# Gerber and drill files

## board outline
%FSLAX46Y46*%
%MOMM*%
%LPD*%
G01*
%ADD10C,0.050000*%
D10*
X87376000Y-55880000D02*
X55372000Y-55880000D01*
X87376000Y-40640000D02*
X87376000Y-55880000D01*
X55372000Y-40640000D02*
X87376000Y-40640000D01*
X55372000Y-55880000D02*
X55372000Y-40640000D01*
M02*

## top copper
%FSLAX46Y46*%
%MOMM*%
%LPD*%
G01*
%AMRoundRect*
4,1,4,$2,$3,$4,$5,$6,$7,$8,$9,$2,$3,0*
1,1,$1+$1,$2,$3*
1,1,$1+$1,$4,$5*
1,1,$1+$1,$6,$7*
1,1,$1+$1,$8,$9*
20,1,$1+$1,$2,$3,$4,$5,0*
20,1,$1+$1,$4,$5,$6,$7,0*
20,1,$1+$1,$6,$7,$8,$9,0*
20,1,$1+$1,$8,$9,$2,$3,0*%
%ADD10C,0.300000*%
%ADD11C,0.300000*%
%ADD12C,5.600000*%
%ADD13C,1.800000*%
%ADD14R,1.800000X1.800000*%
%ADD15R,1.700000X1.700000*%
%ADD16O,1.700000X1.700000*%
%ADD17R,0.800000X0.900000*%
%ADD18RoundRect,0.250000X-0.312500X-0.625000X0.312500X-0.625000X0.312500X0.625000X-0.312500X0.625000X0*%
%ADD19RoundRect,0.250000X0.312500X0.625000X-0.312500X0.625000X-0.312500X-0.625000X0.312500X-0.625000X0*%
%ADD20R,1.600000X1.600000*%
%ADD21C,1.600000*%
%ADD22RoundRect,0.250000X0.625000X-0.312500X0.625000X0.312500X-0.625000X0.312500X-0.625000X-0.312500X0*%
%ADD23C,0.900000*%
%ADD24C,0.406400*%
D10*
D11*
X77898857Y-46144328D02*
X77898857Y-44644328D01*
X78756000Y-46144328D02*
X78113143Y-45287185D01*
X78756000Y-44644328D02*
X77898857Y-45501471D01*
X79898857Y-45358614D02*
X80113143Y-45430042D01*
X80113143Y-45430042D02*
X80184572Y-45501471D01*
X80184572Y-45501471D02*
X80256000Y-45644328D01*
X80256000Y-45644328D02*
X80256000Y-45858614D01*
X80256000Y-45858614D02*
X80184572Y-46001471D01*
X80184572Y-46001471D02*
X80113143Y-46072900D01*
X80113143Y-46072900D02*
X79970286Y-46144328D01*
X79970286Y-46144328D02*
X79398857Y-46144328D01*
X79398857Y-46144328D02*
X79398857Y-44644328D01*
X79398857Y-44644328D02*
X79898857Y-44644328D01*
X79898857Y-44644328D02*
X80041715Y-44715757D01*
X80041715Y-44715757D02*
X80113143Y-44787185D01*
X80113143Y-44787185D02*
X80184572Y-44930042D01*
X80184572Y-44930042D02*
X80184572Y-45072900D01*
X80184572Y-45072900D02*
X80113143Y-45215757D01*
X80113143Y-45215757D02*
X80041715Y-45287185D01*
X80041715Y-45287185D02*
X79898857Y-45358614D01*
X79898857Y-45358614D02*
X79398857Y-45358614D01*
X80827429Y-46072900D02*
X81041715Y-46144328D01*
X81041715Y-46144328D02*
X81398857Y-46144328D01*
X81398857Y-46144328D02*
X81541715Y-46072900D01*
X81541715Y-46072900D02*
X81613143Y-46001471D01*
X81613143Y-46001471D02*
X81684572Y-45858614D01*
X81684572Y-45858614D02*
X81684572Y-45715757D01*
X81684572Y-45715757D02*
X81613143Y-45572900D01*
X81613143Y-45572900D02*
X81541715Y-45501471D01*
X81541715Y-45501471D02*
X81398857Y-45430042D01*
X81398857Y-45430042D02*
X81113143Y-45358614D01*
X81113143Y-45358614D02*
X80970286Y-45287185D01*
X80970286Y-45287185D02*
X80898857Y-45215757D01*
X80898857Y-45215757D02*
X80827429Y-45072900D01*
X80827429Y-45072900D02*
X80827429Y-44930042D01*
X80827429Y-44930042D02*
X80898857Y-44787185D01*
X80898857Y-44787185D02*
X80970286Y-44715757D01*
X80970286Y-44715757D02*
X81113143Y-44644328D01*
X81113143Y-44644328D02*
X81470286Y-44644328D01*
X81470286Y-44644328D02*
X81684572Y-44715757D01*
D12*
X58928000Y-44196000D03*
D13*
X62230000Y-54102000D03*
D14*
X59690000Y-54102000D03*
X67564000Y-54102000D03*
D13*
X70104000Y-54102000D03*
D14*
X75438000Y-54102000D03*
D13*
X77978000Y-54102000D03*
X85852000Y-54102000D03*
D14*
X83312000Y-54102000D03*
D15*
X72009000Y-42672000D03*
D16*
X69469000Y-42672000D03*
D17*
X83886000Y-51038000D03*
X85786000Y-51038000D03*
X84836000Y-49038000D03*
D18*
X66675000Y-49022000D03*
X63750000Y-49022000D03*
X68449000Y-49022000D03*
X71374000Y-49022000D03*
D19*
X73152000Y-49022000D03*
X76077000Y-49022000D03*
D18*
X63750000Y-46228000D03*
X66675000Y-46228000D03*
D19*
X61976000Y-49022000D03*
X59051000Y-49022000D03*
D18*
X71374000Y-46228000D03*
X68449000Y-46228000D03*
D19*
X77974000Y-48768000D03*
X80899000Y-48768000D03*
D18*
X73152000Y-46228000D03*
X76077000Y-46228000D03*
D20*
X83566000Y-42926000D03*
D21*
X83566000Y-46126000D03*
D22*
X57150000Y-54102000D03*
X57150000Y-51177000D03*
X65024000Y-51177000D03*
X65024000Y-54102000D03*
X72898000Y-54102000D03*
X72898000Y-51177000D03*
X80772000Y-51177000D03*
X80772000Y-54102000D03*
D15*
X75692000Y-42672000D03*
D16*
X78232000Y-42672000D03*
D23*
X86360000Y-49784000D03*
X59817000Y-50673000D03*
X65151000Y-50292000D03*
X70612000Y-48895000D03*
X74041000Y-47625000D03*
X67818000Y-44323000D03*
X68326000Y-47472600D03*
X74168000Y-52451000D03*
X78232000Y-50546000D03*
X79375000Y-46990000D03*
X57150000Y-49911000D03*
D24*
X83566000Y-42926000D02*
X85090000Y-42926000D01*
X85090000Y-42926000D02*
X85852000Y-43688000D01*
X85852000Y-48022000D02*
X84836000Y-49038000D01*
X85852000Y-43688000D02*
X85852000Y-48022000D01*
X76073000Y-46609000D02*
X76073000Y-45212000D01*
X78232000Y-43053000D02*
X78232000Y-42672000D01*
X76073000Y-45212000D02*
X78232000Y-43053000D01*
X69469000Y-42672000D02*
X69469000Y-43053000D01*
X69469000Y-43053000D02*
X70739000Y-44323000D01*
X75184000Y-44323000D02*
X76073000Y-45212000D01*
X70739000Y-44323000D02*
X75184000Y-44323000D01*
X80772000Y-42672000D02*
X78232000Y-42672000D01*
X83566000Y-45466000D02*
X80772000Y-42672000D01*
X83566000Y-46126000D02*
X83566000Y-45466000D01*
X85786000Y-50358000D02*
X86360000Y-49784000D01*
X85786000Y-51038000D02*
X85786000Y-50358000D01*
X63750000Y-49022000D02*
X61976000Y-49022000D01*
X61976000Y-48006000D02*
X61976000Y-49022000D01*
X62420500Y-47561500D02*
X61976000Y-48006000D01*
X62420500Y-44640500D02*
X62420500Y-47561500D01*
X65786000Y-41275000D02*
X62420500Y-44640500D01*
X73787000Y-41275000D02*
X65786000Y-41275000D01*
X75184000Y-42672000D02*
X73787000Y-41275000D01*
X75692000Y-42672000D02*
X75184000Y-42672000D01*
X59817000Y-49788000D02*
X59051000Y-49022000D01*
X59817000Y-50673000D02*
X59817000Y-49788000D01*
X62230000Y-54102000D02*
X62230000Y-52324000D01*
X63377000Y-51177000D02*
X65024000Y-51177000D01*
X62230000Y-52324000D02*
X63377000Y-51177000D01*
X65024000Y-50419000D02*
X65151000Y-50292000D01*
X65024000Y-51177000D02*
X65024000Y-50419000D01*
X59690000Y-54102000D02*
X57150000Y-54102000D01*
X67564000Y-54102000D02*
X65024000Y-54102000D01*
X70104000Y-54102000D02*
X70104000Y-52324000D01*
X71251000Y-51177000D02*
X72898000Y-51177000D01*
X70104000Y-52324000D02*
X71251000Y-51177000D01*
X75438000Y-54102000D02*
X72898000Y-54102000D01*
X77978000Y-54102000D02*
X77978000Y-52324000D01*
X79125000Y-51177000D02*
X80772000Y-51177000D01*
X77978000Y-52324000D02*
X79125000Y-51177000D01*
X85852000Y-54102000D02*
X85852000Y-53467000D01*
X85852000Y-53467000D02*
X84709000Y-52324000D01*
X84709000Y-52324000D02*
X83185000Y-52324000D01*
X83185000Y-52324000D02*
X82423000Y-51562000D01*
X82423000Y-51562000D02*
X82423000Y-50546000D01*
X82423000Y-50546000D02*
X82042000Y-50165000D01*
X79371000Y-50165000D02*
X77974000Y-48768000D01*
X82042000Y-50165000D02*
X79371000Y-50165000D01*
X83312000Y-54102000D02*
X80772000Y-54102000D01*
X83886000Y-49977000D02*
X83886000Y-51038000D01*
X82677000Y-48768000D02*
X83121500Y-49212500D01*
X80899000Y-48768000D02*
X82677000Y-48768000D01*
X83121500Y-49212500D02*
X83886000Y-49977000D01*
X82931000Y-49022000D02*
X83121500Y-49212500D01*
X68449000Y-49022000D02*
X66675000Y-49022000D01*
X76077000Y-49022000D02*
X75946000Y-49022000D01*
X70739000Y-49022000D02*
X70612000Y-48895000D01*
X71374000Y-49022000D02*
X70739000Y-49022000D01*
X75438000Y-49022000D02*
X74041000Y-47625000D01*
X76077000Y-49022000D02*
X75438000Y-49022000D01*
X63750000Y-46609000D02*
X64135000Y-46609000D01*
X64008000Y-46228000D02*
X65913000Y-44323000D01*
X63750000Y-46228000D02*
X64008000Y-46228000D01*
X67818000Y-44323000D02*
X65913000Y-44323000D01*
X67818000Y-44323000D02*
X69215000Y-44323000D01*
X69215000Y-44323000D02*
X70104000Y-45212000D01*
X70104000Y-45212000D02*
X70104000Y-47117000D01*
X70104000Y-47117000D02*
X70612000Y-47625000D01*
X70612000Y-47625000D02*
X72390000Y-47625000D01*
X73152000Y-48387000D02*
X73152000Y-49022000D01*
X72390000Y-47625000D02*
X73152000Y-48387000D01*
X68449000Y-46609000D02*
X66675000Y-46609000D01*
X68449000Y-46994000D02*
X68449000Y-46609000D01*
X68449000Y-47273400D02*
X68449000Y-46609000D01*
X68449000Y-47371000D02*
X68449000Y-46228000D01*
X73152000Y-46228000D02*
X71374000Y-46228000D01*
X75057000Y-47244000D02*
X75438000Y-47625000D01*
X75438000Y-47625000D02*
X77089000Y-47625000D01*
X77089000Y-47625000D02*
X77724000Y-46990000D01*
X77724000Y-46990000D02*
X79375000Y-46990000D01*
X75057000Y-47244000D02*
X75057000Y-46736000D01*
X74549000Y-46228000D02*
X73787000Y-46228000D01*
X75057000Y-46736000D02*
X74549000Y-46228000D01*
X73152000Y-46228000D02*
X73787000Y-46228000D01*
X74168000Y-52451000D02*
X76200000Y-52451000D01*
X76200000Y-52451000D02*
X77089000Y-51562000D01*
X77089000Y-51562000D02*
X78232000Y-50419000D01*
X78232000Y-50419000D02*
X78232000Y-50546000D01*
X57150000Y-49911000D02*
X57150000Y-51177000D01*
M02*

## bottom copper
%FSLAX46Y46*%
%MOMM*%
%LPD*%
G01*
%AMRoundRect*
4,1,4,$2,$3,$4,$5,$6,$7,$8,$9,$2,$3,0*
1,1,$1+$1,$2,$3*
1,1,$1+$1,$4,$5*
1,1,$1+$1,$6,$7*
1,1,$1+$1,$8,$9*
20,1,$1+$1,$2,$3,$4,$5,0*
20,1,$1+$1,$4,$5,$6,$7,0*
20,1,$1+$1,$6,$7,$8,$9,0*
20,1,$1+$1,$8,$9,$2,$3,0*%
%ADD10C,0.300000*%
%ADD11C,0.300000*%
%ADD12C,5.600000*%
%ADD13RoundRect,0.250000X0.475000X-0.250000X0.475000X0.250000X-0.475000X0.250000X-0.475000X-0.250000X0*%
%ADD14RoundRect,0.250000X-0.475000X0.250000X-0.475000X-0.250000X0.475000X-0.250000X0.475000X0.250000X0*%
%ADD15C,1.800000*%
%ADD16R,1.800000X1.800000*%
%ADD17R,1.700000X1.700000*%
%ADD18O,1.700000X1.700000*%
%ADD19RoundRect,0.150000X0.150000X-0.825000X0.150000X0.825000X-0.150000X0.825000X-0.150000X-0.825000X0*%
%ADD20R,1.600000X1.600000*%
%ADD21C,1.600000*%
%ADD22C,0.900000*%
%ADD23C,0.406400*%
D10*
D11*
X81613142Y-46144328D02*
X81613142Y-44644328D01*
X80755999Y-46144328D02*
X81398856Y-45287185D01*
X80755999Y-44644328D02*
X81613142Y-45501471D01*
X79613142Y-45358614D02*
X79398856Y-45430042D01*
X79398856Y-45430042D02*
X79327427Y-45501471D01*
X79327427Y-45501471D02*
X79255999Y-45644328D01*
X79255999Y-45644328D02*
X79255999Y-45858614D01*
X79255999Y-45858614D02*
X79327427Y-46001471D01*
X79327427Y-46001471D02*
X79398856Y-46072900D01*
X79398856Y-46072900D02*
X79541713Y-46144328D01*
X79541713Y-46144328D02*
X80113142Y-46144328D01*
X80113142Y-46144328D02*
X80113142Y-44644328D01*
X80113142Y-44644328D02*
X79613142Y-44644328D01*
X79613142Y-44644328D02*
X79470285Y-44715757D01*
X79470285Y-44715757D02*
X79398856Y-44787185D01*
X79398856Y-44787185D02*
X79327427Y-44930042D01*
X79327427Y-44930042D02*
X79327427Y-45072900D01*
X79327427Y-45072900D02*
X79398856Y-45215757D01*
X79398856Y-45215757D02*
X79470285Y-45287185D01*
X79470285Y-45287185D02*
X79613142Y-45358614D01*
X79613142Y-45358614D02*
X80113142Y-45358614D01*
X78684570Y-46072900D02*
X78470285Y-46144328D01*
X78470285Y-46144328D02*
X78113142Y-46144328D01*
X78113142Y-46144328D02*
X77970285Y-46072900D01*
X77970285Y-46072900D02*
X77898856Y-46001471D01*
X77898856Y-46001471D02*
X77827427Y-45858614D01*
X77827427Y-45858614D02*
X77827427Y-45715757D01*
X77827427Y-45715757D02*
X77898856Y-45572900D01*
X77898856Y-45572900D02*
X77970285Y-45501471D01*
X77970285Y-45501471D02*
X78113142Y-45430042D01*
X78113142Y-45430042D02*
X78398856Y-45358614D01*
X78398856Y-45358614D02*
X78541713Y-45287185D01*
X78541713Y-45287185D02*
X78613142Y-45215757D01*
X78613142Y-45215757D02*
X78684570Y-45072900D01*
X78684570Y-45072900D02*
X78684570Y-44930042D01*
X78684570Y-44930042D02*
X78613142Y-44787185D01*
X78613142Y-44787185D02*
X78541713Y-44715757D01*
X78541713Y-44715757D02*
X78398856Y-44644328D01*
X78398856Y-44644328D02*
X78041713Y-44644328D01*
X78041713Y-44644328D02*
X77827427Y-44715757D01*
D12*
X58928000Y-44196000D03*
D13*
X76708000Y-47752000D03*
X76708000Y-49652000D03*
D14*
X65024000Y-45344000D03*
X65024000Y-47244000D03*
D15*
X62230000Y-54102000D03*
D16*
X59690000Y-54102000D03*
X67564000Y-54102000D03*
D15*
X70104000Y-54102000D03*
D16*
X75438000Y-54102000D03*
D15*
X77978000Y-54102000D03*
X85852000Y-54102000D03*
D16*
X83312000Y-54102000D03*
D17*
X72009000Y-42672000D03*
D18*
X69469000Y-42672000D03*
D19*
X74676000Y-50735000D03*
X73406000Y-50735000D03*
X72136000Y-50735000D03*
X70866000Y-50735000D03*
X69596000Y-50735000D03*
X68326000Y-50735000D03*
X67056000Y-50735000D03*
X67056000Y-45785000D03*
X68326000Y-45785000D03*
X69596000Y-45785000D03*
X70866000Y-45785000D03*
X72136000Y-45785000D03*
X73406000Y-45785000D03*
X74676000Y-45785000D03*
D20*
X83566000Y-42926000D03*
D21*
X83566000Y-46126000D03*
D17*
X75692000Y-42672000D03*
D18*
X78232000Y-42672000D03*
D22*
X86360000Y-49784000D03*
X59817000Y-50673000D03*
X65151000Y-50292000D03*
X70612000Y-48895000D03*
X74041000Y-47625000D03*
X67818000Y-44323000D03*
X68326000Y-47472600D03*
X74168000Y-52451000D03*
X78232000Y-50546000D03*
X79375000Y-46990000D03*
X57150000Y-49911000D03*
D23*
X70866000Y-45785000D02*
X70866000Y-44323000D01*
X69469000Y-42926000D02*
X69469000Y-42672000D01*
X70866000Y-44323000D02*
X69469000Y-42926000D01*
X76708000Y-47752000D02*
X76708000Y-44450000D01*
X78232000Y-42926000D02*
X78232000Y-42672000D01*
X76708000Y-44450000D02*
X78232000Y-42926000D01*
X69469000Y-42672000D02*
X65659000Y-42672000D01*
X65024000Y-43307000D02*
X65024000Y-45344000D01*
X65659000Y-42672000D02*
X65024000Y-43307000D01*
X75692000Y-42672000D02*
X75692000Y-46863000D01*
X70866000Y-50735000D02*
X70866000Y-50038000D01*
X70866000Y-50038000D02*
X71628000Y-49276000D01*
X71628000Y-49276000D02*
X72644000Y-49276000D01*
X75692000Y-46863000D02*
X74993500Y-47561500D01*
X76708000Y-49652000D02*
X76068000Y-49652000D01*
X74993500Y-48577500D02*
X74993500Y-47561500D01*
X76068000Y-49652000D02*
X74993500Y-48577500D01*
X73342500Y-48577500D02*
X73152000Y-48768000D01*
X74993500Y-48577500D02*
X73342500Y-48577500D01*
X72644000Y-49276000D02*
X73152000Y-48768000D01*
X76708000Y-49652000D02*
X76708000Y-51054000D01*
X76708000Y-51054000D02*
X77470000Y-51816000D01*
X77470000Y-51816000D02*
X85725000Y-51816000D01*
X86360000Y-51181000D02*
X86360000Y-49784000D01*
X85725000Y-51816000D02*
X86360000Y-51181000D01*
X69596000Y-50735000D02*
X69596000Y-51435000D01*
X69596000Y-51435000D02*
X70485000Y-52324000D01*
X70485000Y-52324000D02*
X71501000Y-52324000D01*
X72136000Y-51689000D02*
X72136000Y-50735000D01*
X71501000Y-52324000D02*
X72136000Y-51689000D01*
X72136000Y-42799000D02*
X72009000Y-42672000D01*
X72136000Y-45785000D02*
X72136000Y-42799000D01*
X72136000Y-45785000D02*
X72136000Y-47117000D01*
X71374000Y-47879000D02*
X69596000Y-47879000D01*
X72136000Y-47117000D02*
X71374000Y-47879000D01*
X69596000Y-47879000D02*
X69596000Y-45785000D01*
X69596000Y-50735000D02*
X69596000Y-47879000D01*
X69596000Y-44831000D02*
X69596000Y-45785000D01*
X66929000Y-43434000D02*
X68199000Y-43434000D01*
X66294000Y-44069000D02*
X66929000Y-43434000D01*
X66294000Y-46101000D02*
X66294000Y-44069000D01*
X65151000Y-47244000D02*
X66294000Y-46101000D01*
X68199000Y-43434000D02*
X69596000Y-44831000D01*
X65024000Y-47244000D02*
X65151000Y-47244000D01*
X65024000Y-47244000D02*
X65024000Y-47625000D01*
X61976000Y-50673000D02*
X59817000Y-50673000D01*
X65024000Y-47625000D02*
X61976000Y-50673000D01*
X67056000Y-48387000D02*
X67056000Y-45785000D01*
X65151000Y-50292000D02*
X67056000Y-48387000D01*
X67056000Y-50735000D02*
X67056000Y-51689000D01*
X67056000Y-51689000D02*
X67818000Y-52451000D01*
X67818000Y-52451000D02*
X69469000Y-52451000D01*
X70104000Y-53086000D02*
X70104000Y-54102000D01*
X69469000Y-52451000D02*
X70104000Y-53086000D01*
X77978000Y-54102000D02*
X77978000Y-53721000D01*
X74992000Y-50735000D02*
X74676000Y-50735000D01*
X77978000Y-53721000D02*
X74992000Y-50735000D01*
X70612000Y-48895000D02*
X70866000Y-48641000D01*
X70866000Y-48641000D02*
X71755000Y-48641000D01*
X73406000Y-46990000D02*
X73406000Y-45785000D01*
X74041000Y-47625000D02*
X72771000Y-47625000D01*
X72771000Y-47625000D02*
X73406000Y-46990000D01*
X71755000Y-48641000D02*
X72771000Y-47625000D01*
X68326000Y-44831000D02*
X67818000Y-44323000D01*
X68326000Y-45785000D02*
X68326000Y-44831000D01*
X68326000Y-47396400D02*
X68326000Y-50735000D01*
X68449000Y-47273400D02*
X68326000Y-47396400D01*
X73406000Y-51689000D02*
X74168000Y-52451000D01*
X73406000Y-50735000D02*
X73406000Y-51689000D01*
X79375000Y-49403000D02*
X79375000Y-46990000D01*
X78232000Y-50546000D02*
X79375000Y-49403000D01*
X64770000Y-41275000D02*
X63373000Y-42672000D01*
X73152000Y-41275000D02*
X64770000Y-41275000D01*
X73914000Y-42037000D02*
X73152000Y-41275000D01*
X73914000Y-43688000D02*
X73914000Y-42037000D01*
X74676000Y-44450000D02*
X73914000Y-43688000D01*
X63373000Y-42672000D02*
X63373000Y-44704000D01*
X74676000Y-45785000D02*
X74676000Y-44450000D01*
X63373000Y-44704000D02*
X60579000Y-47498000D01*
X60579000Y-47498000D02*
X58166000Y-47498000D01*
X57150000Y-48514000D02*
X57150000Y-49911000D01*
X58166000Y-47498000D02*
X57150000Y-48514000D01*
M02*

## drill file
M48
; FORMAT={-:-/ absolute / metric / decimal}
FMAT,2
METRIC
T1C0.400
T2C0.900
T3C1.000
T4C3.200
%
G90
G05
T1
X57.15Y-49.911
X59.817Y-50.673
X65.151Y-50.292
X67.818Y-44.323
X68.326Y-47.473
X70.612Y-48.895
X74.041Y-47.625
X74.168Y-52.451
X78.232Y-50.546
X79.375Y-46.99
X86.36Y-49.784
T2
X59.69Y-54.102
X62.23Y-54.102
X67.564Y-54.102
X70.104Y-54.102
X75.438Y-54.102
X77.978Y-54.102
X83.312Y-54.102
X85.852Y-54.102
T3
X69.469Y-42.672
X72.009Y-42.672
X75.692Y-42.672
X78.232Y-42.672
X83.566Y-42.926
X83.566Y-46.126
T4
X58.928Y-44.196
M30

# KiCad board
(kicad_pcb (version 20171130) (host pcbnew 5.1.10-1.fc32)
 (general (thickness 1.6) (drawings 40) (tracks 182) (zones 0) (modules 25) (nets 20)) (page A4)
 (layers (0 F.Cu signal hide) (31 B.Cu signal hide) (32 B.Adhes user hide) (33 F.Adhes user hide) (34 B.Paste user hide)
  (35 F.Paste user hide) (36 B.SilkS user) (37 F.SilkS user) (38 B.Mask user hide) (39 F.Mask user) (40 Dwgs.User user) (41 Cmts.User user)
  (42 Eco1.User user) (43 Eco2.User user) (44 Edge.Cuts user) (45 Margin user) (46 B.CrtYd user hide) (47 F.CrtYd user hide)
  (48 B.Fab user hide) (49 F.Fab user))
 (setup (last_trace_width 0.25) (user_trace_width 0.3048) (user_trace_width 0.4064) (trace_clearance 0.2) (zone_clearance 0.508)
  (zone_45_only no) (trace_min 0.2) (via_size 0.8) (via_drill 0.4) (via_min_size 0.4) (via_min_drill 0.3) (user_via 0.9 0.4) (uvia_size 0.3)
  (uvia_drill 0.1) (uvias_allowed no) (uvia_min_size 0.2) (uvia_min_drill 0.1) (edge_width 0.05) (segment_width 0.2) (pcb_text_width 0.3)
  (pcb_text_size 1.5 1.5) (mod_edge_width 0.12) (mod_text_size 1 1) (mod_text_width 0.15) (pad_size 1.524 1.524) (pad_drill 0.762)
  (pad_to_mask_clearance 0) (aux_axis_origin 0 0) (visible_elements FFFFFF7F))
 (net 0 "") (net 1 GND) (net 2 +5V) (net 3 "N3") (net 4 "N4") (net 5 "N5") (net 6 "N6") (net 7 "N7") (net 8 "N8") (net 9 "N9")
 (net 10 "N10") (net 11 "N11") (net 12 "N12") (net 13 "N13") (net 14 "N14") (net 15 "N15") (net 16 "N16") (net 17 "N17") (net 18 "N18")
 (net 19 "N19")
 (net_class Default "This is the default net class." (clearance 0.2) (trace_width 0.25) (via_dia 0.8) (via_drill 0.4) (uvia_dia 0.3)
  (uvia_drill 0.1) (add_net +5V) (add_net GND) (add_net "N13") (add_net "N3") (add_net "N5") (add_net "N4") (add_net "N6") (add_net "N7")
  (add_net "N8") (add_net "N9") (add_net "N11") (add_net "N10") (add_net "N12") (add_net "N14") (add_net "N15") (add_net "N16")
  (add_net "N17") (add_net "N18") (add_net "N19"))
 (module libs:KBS (layer B.Cu) (at 60.071 48.895 180)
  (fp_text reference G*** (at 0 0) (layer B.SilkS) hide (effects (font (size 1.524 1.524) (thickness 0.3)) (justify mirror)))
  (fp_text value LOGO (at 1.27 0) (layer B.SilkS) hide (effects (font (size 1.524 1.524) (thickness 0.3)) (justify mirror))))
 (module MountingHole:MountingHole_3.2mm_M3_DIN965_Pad (layer F.Cu) (at 58.928 44.196)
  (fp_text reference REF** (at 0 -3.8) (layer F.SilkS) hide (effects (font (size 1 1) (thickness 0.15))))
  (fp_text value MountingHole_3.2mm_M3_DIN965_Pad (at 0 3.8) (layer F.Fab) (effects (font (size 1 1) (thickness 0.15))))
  (pad 1 thru_hole circle (at 0 0) (size 5.6 5.6) (drill 3.2) (layers *.Cu *.Mask)))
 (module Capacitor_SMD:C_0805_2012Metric (layer B.Cu) (at 76.708 48.702 90)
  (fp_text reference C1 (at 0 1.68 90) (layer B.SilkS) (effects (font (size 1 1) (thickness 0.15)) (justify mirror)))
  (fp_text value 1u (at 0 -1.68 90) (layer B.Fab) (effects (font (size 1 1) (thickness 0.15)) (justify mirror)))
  (pad 2 smd roundrect (at 0.95 0 90) (size 1 1.45) (layers B.Cu B.Paste B.Mask) (roundrect_rratio 0.25) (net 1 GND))
  (pad 1 smd roundrect (at -0.95 0 90) (size 1 1.45) (layers B.Cu B.Paste B.Mask) (roundrect_rratio 0.25) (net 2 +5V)))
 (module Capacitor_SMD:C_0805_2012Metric (layer B.Cu) (at 65.024 46.294 270)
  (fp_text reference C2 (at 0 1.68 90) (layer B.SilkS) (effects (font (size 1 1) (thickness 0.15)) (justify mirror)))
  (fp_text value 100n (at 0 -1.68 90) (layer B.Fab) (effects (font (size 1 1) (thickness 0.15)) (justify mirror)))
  (pad 1 smd roundrect (at -0.95 0 270) (size 1 1.45) (layers B.Cu B.Paste B.Mask) (roundrect_rratio 0.25) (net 1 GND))
  (pad 2 smd roundrect (at 0.95 0 270) (size 1 1.45) (layers B.Cu B.Paste B.Mask) (roundrect_rratio 0.25) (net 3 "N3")))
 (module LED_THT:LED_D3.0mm (layer F.Cu) (at 59.69 54.102)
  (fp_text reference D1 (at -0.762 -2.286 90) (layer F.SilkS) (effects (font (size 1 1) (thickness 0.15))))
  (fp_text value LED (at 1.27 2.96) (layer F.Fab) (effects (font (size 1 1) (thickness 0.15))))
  (pad 2 thru_hole circle (at 2.54 0) (size 1.8 1.8) (drill 0.9) (layers *.Cu *.Mask) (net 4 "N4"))
  (pad 1 thru_hole rect (at 0 0) (size 1.8 1.8) (drill 0.9) (layers *.Cu *.Mask) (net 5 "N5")))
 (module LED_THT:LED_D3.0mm (layer F.Cu) (at 67.564 54.102)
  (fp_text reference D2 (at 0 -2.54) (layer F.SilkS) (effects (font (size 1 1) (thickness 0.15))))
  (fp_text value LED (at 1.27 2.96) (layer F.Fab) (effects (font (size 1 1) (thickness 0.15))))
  (pad 1 thru_hole rect (at 0 0) (size 1.8 1.8) (drill 0.9) (layers *.Cu *.Mask) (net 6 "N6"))
  (pad 2 thru_hole circle (at 2.54 0) (size 1.8 1.8) (drill 0.9) (layers *.Cu *.Mask) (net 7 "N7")))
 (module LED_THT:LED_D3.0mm (layer F.Cu) (at 75.438 54.102)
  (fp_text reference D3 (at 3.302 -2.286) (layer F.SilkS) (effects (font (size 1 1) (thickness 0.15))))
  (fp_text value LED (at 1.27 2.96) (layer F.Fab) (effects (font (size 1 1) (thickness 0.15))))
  (pad 1 thru_hole rect (at 0 0) (size 1.8 1.8) (drill 0.9) (layers *.Cu *.Mask) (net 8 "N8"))
  (pad 2 thru_hole circle (at 2.54 0) (size 1.8 1.8) (drill 0.9) (layers *.Cu *.Mask) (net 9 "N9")))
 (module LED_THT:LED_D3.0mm (layer F.Cu) (at 83.312 54.102)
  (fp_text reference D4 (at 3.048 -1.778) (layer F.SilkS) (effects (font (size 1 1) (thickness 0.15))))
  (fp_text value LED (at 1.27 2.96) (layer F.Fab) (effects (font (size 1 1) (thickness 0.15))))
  (pad 2 thru_hole circle (at 2.54 0) (size 1.8 1.8) (drill 0.9) (layers *.Cu *.Mask) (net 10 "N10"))
  (pad 1 thru_hole rect (at 0 0) (size 1.8 1.8) (drill 0.9) (layers *.Cu *.Mask) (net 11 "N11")))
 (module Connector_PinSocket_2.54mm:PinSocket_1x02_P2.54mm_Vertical (layer F.Cu) (at 72.009 42.672 270)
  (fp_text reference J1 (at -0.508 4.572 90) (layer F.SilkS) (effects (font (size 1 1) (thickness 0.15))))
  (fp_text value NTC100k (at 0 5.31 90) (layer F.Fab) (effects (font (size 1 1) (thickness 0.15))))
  (pad 1 thru_hole rect (at 0 0 270) (size 1.7 1.7) (drill 1) (layers *.Cu *.Mask) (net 3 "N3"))
  (pad 2 thru_hole oval (at 0 2.54 270) (size 1.7 1.7) (drill 1) (layers *.Cu *.Mask) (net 1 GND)))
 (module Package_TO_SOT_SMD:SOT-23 (layer F.Cu) (at 84.836 50.038 90)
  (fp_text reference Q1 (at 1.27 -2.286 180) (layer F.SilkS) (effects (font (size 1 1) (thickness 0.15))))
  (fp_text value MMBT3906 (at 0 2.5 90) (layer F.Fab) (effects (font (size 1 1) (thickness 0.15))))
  (pad 1 smd rect (at -1 -0.95 90) (size 0.9 0.8) (layers F.Cu F.Paste F.Mask) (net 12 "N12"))
  (pad 2 smd rect (at -1 0.95 90) (size 0.9 0.8) (layers F.Cu F.Paste F.Mask) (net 2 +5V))
  (pad 3 smd rect (at 1 0 90) (size 0.9 0.8) (layers F.Cu F.Paste F.Mask) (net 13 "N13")))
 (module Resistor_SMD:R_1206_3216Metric (layer F.Cu) (at 65.2125 49.022)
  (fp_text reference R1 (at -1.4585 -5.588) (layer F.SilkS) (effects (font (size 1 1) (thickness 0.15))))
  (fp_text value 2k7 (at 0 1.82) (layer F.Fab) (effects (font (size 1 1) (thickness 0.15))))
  (pad 2 smd roundrect (at 1.4625 0) (size 1.125 1.75) (layers F.Cu F.Paste F.Mask) (roundrect_rratio 0.222222) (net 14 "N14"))
  (pad 1 smd roundrect (at -1.4625 0) (size 1.125 1.75) (layers F.Cu F.Paste F.Mask) (roundrect_rratio 0.222222) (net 2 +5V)))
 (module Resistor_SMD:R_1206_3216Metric (layer F.Cu) (at 69.9115 49.022)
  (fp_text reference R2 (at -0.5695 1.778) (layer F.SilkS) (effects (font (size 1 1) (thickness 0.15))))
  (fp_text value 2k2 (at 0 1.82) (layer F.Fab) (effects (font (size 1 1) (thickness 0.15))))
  (pad 1 smd roundrect (at -1.4625 0) (size 1.125 1.75) (layers F.Cu F.Paste F.Mask) (roundrect_rratio 0.222222) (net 14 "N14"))
  (pad 2 smd roundrect (at 1.4625 0) (size 1.125 1.75) (layers F.Cu F.Paste F.Mask) (roundrect_rratio 0.222222) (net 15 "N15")))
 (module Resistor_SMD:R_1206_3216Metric (layer F.Cu) (at 74.6145 49.022 180)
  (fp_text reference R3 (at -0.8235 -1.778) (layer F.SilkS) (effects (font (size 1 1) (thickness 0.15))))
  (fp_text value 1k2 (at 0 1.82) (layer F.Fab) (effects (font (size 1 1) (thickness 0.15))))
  (pad 2 smd roundrect (at 1.4625 0 180) (size 1.125 1.75) (layers F.Cu F.Paste F.Mask) (roundrect_rratio 0.222222) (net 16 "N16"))
  (pad 1 smd roundrect (at -1.4625 0 180) (size 1.125 1.75) (layers F.Cu F.Paste F.Mask) (roundrect_rratio 0.222222) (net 15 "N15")))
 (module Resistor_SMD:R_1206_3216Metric (layer F.Cu) (at 65.2125 46.228)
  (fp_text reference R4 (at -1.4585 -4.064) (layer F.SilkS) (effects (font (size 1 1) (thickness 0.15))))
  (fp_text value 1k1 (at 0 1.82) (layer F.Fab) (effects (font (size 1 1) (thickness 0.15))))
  (pad 1 smd roundrect (at -1.4625 0) (size 1.125 1.75) (layers F.Cu F.Paste F.Mask) (roundrect_rratio 0.222222) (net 16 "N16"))
  (pad 2 smd roundrect (at 1.4625 0) (size 1.125 1.75) (layers F.Cu F.Paste F.Mask) (roundrect_rratio 0.222222) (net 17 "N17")))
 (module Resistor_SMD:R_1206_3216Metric (layer F.Cu) (at 60.5135 49.022 180)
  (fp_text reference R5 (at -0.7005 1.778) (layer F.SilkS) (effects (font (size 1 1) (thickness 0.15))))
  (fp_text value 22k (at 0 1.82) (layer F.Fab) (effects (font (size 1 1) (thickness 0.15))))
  (pad 1 smd roundrect (at -1.4625 0 180) (size 1.125 1.75) (layers F.Cu F.Paste F.Mask) (roundrect_rratio 0.222222) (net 2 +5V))
  (pad 2 smd roundrect (at 1.4625 0 180) (size 1.125 1.75) (layers F.Cu F.Paste F.Mask) (roundrect_rratio 0.222222) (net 3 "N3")))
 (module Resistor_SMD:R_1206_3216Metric (layer F.Cu) (at 69.9115 46.228)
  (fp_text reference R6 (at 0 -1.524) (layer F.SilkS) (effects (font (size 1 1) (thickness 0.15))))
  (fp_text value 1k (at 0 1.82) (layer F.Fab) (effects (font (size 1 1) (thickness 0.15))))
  (pad 2 smd roundrect (at 1.4625 0) (size 1.125 1.75) (layers F.Cu F.Paste F.Mask) (roundrect_rratio 0.222222) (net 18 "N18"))
  (pad 1 smd roundrect (at -1.4625 0) (size 1.125 1.75) (layers F.Cu F.Paste F.Mask) (roundrect_rratio 0.222222) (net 17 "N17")))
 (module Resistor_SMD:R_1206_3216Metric (layer F.Cu) (at 79.4365 48.768 180)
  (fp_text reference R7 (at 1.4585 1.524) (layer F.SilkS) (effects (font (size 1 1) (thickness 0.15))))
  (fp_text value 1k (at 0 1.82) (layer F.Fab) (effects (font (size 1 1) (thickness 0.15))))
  (pad 2 smd roundrect (at 1.4625 0 180) (size 1.125 1.75) (layers F.Cu F.Paste F.Mask) (roundrect_rratio 0.222222) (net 10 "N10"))
  (pad 1 smd roundrect (at -1.4625 0 180) (size 1.125 1.75) (layers F.Cu F.Paste F.Mask) (roundrect_rratio 0.222222) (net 12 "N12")))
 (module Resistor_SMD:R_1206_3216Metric (layer F.Cu) (at 74.6145 46.228)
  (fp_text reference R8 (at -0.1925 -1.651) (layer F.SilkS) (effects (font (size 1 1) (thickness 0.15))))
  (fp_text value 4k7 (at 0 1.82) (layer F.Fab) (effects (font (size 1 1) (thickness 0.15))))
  (pad 1 smd roundrect (at -1.4625 0) (size 1.125 1.75) (layers F.Cu F.Paste F.Mask) (roundrect_rratio 0.222222) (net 18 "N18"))
  (pad 2 smd roundrect (at 1.4625 0) (size 1.125 1.75) (layers F.Cu F.Paste F.Mask) (roundrect_rratio 0.222222) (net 1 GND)))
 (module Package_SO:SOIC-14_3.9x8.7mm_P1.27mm (layer B.Cu) (at 70.866 48.26 90)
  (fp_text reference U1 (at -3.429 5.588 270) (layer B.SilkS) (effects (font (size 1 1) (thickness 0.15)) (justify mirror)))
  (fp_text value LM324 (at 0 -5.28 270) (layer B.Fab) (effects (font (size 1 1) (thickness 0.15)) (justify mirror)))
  (pad 1 smd roundrect (at -2.475 3.81 90) (size 1.95 0.6) (layers B.Cu B.Paste B.Mask) (roundrect_rratio 0.25) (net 9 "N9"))
  (pad 2 smd roundrect (at -2.475 2.54 90) (size 1.95 0.6) (layers B.Cu B.Paste B.Mask) (roundrect_rratio 0.25) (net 18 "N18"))
  (pad 3 smd roundrect (at -2.475 1.27 90) (size 1.95 0.6) (layers B.Cu B.Paste B.Mask) (roundrect_rratio 0.25) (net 3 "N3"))
  (pad 4 smd roundrect (at -2.475 0 90) (size 1.95 0.6) (layers B.Cu B.Paste B.Mask) (roundrect_rratio 0.25) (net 2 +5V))
  (pad 5 smd roundrect (at -2.475 -1.27 90) (size 1.95 0.6) (layers B.Cu B.Paste B.Mask) (roundrect_rratio 0.25) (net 3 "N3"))
  (pad 6 smd roundrect (at -2.475 -2.54 90) (size 1.95 0.6) (layers B.Cu B.Paste B.Mask) (roundrect_rratio 0.25) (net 17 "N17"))
  (pad 7 smd roundrect (at -2.475 -3.81 90) (size 1.95 0.6) (layers B.Cu B.Paste B.Mask) (roundrect_rratio 0.25) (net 7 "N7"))
  (pad 8 smd roundrect (at 2.475 -3.81 90) (size 1.95 0.6) (layers B.Cu B.Paste B.Mask) (roundrect_rratio 0.25) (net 4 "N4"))
  (pad 9 smd roundrect (at 2.475 -2.54 90) (size 1.95 0.6) (layers B.Cu B.Paste B.Mask) (roundrect_rratio 0.25) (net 16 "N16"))
  (pad 10 smd roundrect (at 2.475 -1.27 90) (size 1.95 0.6) (layers B.Cu B.Paste B.Mask) (roundrect_rratio 0.25) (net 3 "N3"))
  (pad 11 smd roundrect (at 2.475 0 90) (size 1.95 0.6) (layers B.Cu B.Paste B.Mask) (roundrect_rratio 0.25) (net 1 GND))
  (pad 12 smd roundrect (at 2.475 1.27 90) (size 1.95 0.6) (layers B.Cu B.Paste B.Mask) (roundrect_rratio 0.25) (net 3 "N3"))
  (pad 13 smd roundrect (at 2.475 2.54 90) (size 1.95 0.6) (layers B.Cu B.Paste B.Mask) (roundrect_rratio 0.25) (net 15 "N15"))
  (pad 14 smd roundrect (at 2.475 3.81 90) (size 1.95 0.6) (layers B.Cu B.Paste B.Mask) (roundrect_rratio 0.25) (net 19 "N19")))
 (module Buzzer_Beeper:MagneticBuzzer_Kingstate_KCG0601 (layer F.Cu) (at 83.566 42.926 270)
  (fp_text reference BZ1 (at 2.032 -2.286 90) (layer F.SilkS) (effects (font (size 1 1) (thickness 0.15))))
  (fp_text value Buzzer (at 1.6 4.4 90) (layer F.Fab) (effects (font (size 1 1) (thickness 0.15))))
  (pad 1 thru_hole rect (at 0 0 270) (size 1.6 1.6) (drill 1) (layers *.Cu *.Mask) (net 13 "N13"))
  (pad 2 thru_hole circle (at 3.2 0 270) (size 1.6 1.6) (drill 1) (layers *.Cu *.Mask) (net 1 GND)))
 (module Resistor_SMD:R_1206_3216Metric (layer F.Cu) (at 57.15 52.6395 90)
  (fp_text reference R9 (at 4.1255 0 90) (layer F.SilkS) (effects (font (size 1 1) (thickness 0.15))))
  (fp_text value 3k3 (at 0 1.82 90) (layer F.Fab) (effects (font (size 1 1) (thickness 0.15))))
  (pad 1 smd roundrect (at -1.4625 0 90) (size 1.125 1.75) (layers F.Cu F.Paste F.Mask) (roundrect_rratio 0.222222) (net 5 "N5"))
  (pad 2 smd roundrect (at 1.4625 0 90) (size 1.125 1.75) (layers F.Cu F.Paste F.Mask) (roundrect_rratio 0.222222) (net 19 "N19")))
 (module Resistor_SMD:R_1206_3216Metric (layer F.Cu) (at 65.024 52.6395 90)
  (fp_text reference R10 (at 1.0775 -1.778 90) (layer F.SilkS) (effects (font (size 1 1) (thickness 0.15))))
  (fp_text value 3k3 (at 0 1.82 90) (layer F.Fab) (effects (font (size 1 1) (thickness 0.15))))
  (pad 2 smd roundrect (at 1.4625 0 90) (size 1.125 1.75) (layers F.Cu F.Paste F.Mask) (roundrect_rratio 0.222222) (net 4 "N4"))
  (pad 1 smd roundrect (at -1.4625 0 90) (size 1.125 1.75) (layers F.Cu F.Paste F.Mask) (roundrect_rratio 0.222222) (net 6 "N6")))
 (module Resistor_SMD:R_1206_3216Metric (layer F.Cu) (at 72.898 52.6395 90)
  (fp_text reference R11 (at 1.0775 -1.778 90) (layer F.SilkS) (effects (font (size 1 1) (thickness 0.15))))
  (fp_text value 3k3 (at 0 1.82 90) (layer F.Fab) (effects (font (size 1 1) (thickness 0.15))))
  (pad 1 smd roundrect (at -1.4625 0 90) (size 1.125 1.75) (layers F.Cu F.Paste F.Mask) (roundrect_rratio 0.222222) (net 8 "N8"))
  (pad 2 smd roundrect (at 1.4625 0 90) (size 1.125 1.75) (layers F.Cu F.Paste F.Mask) (roundrect_rratio 0.222222) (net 7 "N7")))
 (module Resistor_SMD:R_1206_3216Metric (layer F.Cu) (at 80.772 52.6395 90)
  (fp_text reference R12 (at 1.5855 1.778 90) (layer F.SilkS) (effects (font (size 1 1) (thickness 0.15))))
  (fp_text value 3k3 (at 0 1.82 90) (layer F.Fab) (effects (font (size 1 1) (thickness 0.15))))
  (pad 2 smd roundrect (at 1.4625 0 90) (size 1.125 1.75) (layers F.Cu F.Paste F.Mask) (roundrect_rratio 0.222222) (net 9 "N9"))
  (pad 1 smd roundrect (at -1.4625 0 90) (size 1.125 1.75) (layers F.Cu F.Paste F.Mask) (roundrect_rratio 0.222222) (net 11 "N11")))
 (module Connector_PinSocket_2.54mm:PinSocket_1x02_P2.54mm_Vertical (layer F.Cu) (at 75.692 42.672 90)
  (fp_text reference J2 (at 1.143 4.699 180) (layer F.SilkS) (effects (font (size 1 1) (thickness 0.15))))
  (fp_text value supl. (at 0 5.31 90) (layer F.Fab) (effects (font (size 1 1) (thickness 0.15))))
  (pad 1 thru_hole rect (at 0 0 90) (size 1.7 1.7) (drill 1) (layers *.Cu *.Mask) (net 2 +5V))
  (pad 2 thru_hole oval (at 0 2.54 90) (size 1.7 1.7) (drill 1) (layers *.Cu *.Mask) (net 1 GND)))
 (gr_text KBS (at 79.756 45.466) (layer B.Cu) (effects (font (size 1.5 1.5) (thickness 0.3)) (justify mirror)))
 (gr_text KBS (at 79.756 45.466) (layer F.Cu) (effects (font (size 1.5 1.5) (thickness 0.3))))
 (gr_line (start 87.376 55.88) (end 55.372 55.88) (layer Edge.Cuts) (width 0.05))
 (gr_line (start 87.376 40.64) (end 87.376 55.88) (layer Edge.Cuts) (width 0.05))
 (gr_line (start 55.372 40.64) (end 87.376 40.64) (layer Edge.Cuts) (width 0.05))
 (gr_line (start 55.372 55.88) (end 55.372 40.64) (layer Edge.Cuts) (width 0.05))
 (segment (start 83.566 42.926) (end 85.09 42.926) (width 0.4064) (layer F.Cu) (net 13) (status 10))
 (segment (start 85.09 42.926) (end 85.852 43.688) (width 0.4064) (layer F.Cu) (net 13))
 (segment (start 85.852 48.022) (end 84.836 49.038) (width 0.4064) (layer F.Cu) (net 13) (status 20))
 (segment (start 85.852 43.688) (end 85.852 48.022) (width 0.4064) (layer F.Cu) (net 13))
 (segment (start 70.866 45.785) (end 70.866 44.323) (width 0.4064) (layer B.Cu) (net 1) (status 10))
 (segment (start 69.469 42.926) (end 69.469 42.672) (width 0.4064) (layer B.Cu) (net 1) (status 30))
 (segment (start 70.866 44.323) (end 69.469 42.926) (width 0.4064) (layer B.Cu) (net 1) (status 20))
 (segment (start 76.708 47.752) (end 76.708 44.45) (width 0.4064) (layer B.Cu) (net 1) (status 10))
 (segment (start 78.232 42.926) (end 78.232 42.672) (width 0.4064) (layer B.Cu) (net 1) (status 30))
 (segment (start 76.708 44.45) (end 78.232 42.926) (width 0.4064) (layer B.Cu) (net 1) (status 20))
 (segment (start 76.073 46.609) (end 76.073 45.212) (width 0.4064) (layer F.Cu) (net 1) (status 10))
 (segment (start 78.232 43.053) (end 78.232 42.672) (width 0.4064) (layer F.Cu) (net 1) (status 30))
 (segment (start 76.073 45.212) (end 78.232 43.053) (width 0.4064) (layer F.Cu) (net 1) (status 20))
 (segment (start 69.469 42.672) (end 69.469 43.053) (width 0.4064) (layer F.Cu) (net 1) (status 30))
 (segment (start 69.469 43.053) (end 70.739 44.323) (width 0.4064) (layer F.Cu) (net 1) (status 10))
 (segment (start 75.184 44.323) (end 76.073 45.212) (width 0.4064) (layer F.Cu) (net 1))
 (segment (start 70.739 44.323) (end 75.184 44.323) (width 0.4064) (layer F.Cu) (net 1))
 (segment (start 69.469 42.672) (end 65.659 42.672) (width 0.4064) (layer B.Cu) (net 1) (status 10))
 (segment (start 65.024 43.307) (end 65.024 45.344) (width 0.4064) (layer B.Cu) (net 1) (status 20))
 (segment (start 65.659 42.672) (end 65.024 43.307) (width 0.4064) (layer B.Cu) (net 1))
 (segment (start 80.772 42.672) (end 78.232 42.672) (width 0.4064) (layer F.Cu) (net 1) (status 20))
 (segment (start 83.566 45.466) (end 80.772 42.672) (width 0.4064) (layer F.Cu) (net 1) (status 10))
 (segment (start 83.566 46.126) (end 83.566 45.466) (width 0.4064) (layer F.Cu) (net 1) (status 30))
 (via (at 86.36 49.784) (size 0.9) (drill 0.4) (layers F.Cu B.Cu) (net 2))
 (segment (start 85.786 50.358) (end 86.36 49.784) (width 0.4064) (layer F.Cu) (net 2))
 (segment (start 85.786 51.038) (end 85.786 50.358) (width 0.4064) (layer F.Cu) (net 2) (status 10))
 (segment (start 75.692 42.672) (end 75.692 46.863) (width 0.4064) (layer B.Cu) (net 2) (status 10))
 (segment (start 63.75 49.022) (end 61.976 49.022) (width 0.4064) (layer F.Cu) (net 2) (status 30))
 (segment (start 70.866 50.735) (end 70.866 50.038) (width 0.4064) (layer B.Cu) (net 2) (status 30))
 (segment (start 70.866 50.038) (end 71.628 49.276) (width 0.4064) (layer B.Cu) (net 2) (status 10))
 (segment (start 71.628 49.276) (end 72.644 49.276) (width 0.4064) (layer B.Cu) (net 2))
 (segment (start 75.692 46.863) (end 74.9935 47.5615) (width 0.4064) (layer B.Cu) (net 2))
 (segment (start 76.708 49.652) (end 76.068 49.652) (width 0.4064) (layer B.Cu) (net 2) (status 30))
 (segment (start 74.9935 48.5775) (end 74.9935 47.5615) (width 0.4064) (layer B.Cu) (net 2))
 (segment (start 76.068 49.652) (end 74.9935 48.5775) (width 0.4064) (layer B.Cu) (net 2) (status 10))
 (segment (start 73.3425 48.5775) (end 73.152 48.768) (width 0.4064) (layer B.Cu) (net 2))
 (segment (start 74.9935 48.5775) (end 73.3425 48.5775) (width 0.4064) (layer B.Cu) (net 2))
 (segment (start 72.644 49.276) (end 73.152 48.768) (width 0.4064) (layer B.Cu) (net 2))
 (segment (start 76.708 49.652) (end 76.708 51.054) (width 0.4064) (layer B.Cu) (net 2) (status 10))
 (segment (start 76.708 51.054) (end 77.47 51.816) (width 0.4064) (layer B.Cu) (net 2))
 (segment (start 77.47 51.816) (end 85.725 51.816) (width 0.4064) (layer B.Cu) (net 2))
 (segment (start 86.36 51.181) (end 86.36 49.784) (width 0.4064) (layer B.Cu) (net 2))
 (segment (start 85.725 51.816) (end 86.36 51.181) (width 0.4064) (layer B.Cu) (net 2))
 (segment (start 61.976 48.006) (end 61.976 49.022) (width 0.4064) (layer F.Cu) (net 2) (status 20))
 (segment (start 62.4205 47.5615) (end 61.976 48.006) (width 0.4064) (layer F.Cu) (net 2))
 (segment (start 62.4205 44.6405) (end 62.4205 47.5615) (width 0.4064) (layer F.Cu) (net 2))
 (segment (start 65.786 41.275) (end 62.4205 44.6405) (width 0.4064) (layer F.Cu) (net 2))
 (segment (start 73.787 41.275) (end 65.786 41.275) (width 0.4064) (layer F.Cu) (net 2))
 (segment (start 75.184 42.672) (end 73.787 41.275) (width 0.4064) (layer F.Cu) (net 2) (status 10))
 (segment (start 75.692 42.672) (end 75.184 42.672) (width 0.4064) (layer F.Cu) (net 2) (status 30))
 (segment (start 69.596 50.735) (end 69.596 51.435) (width 0.4064) (layer B.Cu) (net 3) (status 30))
 (segment (start 69.596 51.435) (end 70.485 52.324) (width 0.4064) (layer B.Cu) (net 3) (status 10))
 (segment (start 70.485 52.324) (end 71.501 52.324) (width 0.4064) (layer B.Cu) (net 3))
 (segment (start 72.136 51.689) (end 72.136 50.735) (width 0.4064) (layer B.Cu) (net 3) (status 30))
 (segment (start 71.501 52.324) (end 72.136 51.689) (width 0.4064) (layer B.Cu) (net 3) (status 20))
 (segment (start 72.136 42.799) (end 72.009 42.672) (width 0.4064) (layer B.Cu) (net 3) (status 30))
 (segment (start 72.136 45.785) (end 72.136 42.799) (width 0.4064) (layer B.Cu) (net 3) (status 30))
 (segment (start 72.136 45.785) (end 72.136 47.117) (width 0.4064) (layer B.Cu) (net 3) (status 10))
 (segment (start 71.374 47.879) (end 69.596 47.879) (width 0.4064) (layer B.Cu) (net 3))
 (segment (start 72.136 47.117) (end 71.374 47.879) (width 0.4064) (layer B.Cu) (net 3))
 (segment (start 69.596 47.879) (end 69.596 45.785) (width 0.4064) (layer B.Cu) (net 3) (status 20))
 (segment (start 69.596 50.735) (end 69.596 47.879) (width 0.4064) (layer B.Cu) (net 3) (status 10))
 (segment (start 69.596 44.831) (end 69.596 45.785) (width 0.4064) (layer B.Cu) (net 3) (status 30))
 (segment (start 66.929 43.434) (end 68.199 43.434) (width 0.4064) (layer B.Cu) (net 3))
 (segment (start 66.294 44.069) (end 66.929 43.434) (width 0.4064) (layer B.Cu) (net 3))
 (segment (start 66.294 46.101) (end 66.294 44.069) (width 0.4064) (layer B.Cu) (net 3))
 (segment (start 65.151 47.244) (end 66.294 46.101) (width 0.4064) (layer B.Cu) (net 3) (status 10))
 (segment (start 68.199 43.434) (end 69.596 44.831) (width 0.4064) (layer B.Cu) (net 3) (status 20))
 (segment (start 65.024 47.244) (end 65.151 47.244) (width 0.4064) (layer B.Cu) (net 3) (status 30))
 (segment (start 65.024 47.244) (end 65.024 47.625) (width 0.4064) (layer B.Cu) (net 3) (status 30))
 (via (at 59.817 50.673) (size 0.9) (drill 0.4) (layers F.Cu B.Cu) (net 3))
 (segment (start 61.976 50.673) (end 59.817 50.673) (width 0.4064) (layer B.Cu) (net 3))
 (segment (start 65.024 47.625) (end 61.976 50.673) (width 0.4064) (layer B.Cu) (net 3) (status 10))
 (segment (start 59.817 49.788) (end 59.051 49.022) (width 0.4064) (layer F.Cu) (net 3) (status 20))
 (segment (start 59.817 50.673) (end 59.817 49.788) (width 0.4064) (layer F.Cu) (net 3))
 (segment (start 62.23 54.102) (end 62.23 52.324) (width 0.4064) (layer F.Cu) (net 4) (status 10))
 (segment (start 63.377 51.177) (end 65.024 51.177) (width 0.4064) (layer F.Cu) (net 4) (status 20))
 (segment (start 62.23 52.324) (end 63.377 51.177) (width 0.4064) (layer F.Cu) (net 4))
 (via (at 65.151 50.292) (size 0.9) (drill 0.4) (layers F.Cu B.Cu) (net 4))
 (segment (start 65.024 50.419) (end 65.151 50.292) (width 0.4064) (layer F.Cu) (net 4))
 (segment (start 65.024 51.177) (end 65.024 50.419) (width 0.4064) (layer F.Cu) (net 4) (status 10))
 (segment (start 67.056 48.387) (end 67.056 45.785) (width 0.4064) (layer B.Cu) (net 4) (status 20))
 (segment (start 65.151 50.292) (end 67.056 48.387) (width 0.4064) (layer B.Cu) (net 4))
 (segment (start 59.69 54.102) (end 57.15 54.102) (width 0.4064) (layer F.Cu) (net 5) (status 30))
 (segment (start 67.564 54.102) (end 65.024 54.102) (width 0.4064) (layer F.Cu) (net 6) (status 30))
 (segment (start 70.104 54.102) (end 70.104 52.324) (width 0.4064) (layer F.Cu) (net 7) (status 10))
 (segment (start 71.251 51.177) (end 72.898 51.177) (width 0.4064) (layer F.Cu) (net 7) (status 20))
 (segment (start 70.104 52.324) (end 71.251 51.177) (width 0.4064) (layer F.Cu) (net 7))
 (segment (start 67.056 50.735) (end 67.056 51.689) (width 0.4064) (layer B.Cu) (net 7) (status 30))
 (segment (start 67.056 51.689) (end 67.818 52.451) (width 0.4064) (layer B.Cu) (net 7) (status 10))
 (segment (start 67.818 52.451) (end 69.469 52.451) (width 0.4064) (layer B.Cu) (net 7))
 (segment (start 70.104 53.086) (end 70.104 54.102) (width 0.4064) (layer B.Cu) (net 7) (status 20))
 (segment (start 69.469 52.451) (end 70.104 53.086) (width 0.4064) (layer B.Cu) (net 7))
 (segment (start 75.438 54.102) (end 72.898 54.102) (width 0.4064) (layer F.Cu) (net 8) (status 30))
 (segment (start 77.978 54.102) (end 77.978 52.324) (width 0.4064) (layer F.Cu) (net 9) (status 10))
 (segment (start 79.125 51.177) (end 80.772 51.177) (width 0.4064) (layer F.Cu) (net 9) (status 20))
 (segment (start 77.978 52.324) (end 79.125 51.177) (width 0.4064) (layer F.Cu) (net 9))
 (segment (start 77.978 54.102) (end 77.978 53.721) (width 0.4064) (layer B.Cu) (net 9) (status 30))
 (segment (start 74.992 50.735) (end 74.676 50.735) (width 0.4064) (layer B.Cu) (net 9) (status 20))
 (segment (start 77.978 53.721) (end 74.992 50.735) (width 0.4064) (layer B.Cu) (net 9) (status 10))
 (segment (start 85.852 54.102) (end 85.852 53.467) (width 0.4064) (layer F.Cu) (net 10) (status 30))
 (segment (start 85.852 53.467) (end 84.709 52.324) (width 0.4064) (layer F.Cu) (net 10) (status 10))
 (segment (start 84.709 52.324) (end 83.185 52.324) (width 0.4064) (layer F.Cu) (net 10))
 (segment (start 83.185 52.324) (end 82.423 51.562) (width 0.4064) (layer F.Cu) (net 10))
 (segment (start 82.423 51.562) (end 82.423 50.546) (width 0.4064) (layer F.Cu) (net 10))
 (segment (start 82.423 50.546) (end 82.042 50.165) (width 0.4064) (layer F.Cu) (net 10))
 (segment (start 79.371 50.165) (end 77.974 48.768) (width 0.4064) (layer F.Cu) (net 10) (status 20))
 (segment (start 82.042 50.165) (end 79.371 50.165) (width 0.4064) (layer F.Cu) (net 10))
 (segment (start 83.312 54.102) (end 80.772 54.102) (width 0.4064) (layer F.Cu) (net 11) (status 30))
 (segment (start 83.886 49.977) (end 83.886 51.038) (width 0.4064) (layer F.Cu) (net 12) (status 20))
 (segment (start 82.677 48.768) (end 83.1215 49.2125) (width 0.4064) (layer F.Cu) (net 12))
 (segment (start 80.899 48.768) (end 82.677 48.768) (width 0.4064) (layer F.Cu) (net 12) (status 10))
 (segment (start 83.1215 49.2125) (end 83.886 49.977) (width 0.4064) (layer F.Cu) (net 12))
 (segment (start 82.931 49.022) (end 83.1215 49.2125) (width 0.4064) (layer F.Cu) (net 12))
 (segment (start 68.449 49.022) (end 66.675 49.022) (width 0.4064) (layer F.Cu) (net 14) (status 30))
 (segment (start 76.077 49.022) (end 75.946 49.022) (width 0.4064) (layer F.Cu) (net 15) (status 30))
 (via (at 70.612 48.895) (size 0.9) (drill 0.4) (layers F.Cu B.Cu) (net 15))
 (segment (start 70.739 49.022) (end 70.612 48.895) (width 0.4064) (layer F.Cu) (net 15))
 (segment (start 71.374 49.022) (end 70.739 49.022) (width 0.4064) (layer F.Cu) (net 15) (status 10))
 (segment (start 70.612 48.895) (end 70.866 48.641) (width 0.4064) (layer B.Cu) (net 15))
 (segment (start 70.866 48.641) (end 71.755 48.641) (width 0.4064) (layer B.Cu) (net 15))
 (segment (start 73.406 46.99) (end 73.406 45.785) (width 0.4064) (layer B.Cu) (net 15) (status 20))
 (segment (start 75.438 49.022) (end 74.041 47.625) (width 0.4064) (layer F.Cu) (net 15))
 (via (at 74.041 47.625) (size 0.9) (drill 0.4) (layers F.Cu B.Cu) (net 15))
 (segment (start 76.077 49.022) (end 75.438 49.022) (width 0.4064) (layer F.Cu) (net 15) (status 10))
 (segment (start 74.041 47.625) (end 72.771 47.625) (width 0.4064) (layer B.Cu) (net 15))
 (segment (start 72.771 47.625) (end 73.406 46.99) (width 0.4064) (layer B.Cu) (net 15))
 (segment (start 71.755 48.641) (end 72.771 47.625) (width 0.4064) (layer B.Cu) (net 15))
 (segment (start 63.75 46.609) (end 64.135 46.609) (width 0.4064) (layer F.Cu) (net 16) (status 30))
 (via (at 67.818 44.323) (size 0.9) (drill 0.4) (layers F.Cu B.Cu) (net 16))
 (segment (start 68.326 44.831) (end 67.818 44.323) (width 0.4064) (layer B.Cu) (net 16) (status 10))
 (segment (start 68.326 45.785) (end 68.326 44.831) (width 0.4064) (layer B.Cu) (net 16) (status 30))
 (segment (start 64.008 46.228) (end 65.913 44.323) (width 0.4064) (layer F.Cu) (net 16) (status 10))
 (segment (start 63.75 46.228) (end 64.008 46.228) (width 0.4064) (layer F.Cu) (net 16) (status 30))
 (segment (start 67.818 44.323) (end 65.913 44.323) (width 0.4064) (layer F.Cu) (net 16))
 (segment (start 67.818 44.323) (end 69.215 44.323) (width 0.4064) (layer F.Cu) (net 16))
 (segment (start 69.215 44.323) (end 70.104 45.212) (width 0.4064) (layer F.Cu) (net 16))
 (segment (start 70.104 45.212) (end 70.104 47.117) (width 0.4064) (layer F.Cu) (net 16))
 (segment (start 70.104 47.117) (end 70.612 47.625) (width 0.4064) (layer F.Cu) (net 16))
 (segment (start 70.612 47.625) (end 72.39 47.625) (width 0.4064) (layer F.Cu) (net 16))
 (segment (start 73.152 48.387) (end 73.152 49.022) (width 0.4064) (layer F.Cu) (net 16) (status 30))
 (segment (start 72.39 47.625) (end 73.152 48.387) (width 0.4064) (layer F.Cu) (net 16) (status 20))
 (segment (start 68.449 46.609) (end 66.675 46.609) (width 0.4064) (layer F.Cu) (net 17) (status 30))
 (segment (start 68.449 46.994) (end 68.449 46.609) (width 0.4064) (layer F.Cu) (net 17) (status 30))
 (segment (start 68.326 47.3964) (end 68.326 50.735) (width 0.4064) (layer B.Cu) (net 17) (status 20))
 (segment (start 68.449 47.2734) (end 68.449 46.609) (width 0.4064) (layer F.Cu) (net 17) (status 20))
 (segment (start 68.449 47.2734) (end 68.326 47.3964) (width 0.4064) (layer B.Cu) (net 17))
 (via (at 68.326 47.4726) (size 0.9) (drill 0.4) (layers F.Cu B.Cu) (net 17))
 (segment (start 68.449 47.371) (end 68.449 46.228) (width 0.4064) (layer F.Cu) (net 17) (status 20))
 (segment (start 73.152 46.228) (end 71.374 46.228) (width 0.4064) (layer F.Cu) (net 18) (status 30))
 (segment (start 75.057 47.244) (end 75.438 47.625) (width 0.4064) (layer F.Cu) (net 18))
 (segment (start 75.438 47.625) (end 77.089 47.625) (width 0.4064) (layer F.Cu) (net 18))
 (segment (start 77.089 47.625) (end 77.724 46.99) (width 0.4064) (layer F.Cu) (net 18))
 (segment (start 77.724 46.99) (end 79.375 46.99) (width 0.4064) (layer F.Cu) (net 18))
 (segment (start 75.057 47.244) (end 75.057 46.736) (width 0.4064) (layer F.Cu) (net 18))
 (segment (start 74.549 46.228) (end 73.787 46.228) (width 0.4064) (layer F.Cu) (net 18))
 (segment (start 75.057 46.736) (end 74.549 46.228) (width 0.4064) (layer F.Cu) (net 18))
 (segment (start 73.152 46.228) (end 73.787 46.228) (width 0.4064) (layer F.Cu) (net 18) (status 10))
 (via (at 74.168 52.451) (size 0.9) (drill 0.4) (layers F.Cu B.Cu) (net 18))
 (segment (start 73.406 51.689) (end 74.168 52.451) (width 0.4064) (layer B.Cu) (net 18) (status 10))
 (segment (start 73.406 50.735) (end 73.406 51.689) (width 0.4064) (layer B.Cu) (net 18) (status 30))
 (segment (start 74.168 52.451) (end 76.2 52.451) (width 0.4064) (layer F.Cu) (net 18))
 (segment (start 76.2 52.451) (end 77.089 51.562) (width 0.4064) (layer F.Cu) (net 18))
 (segment (start 77.089 51.562) (end 78.232 50.419) (width 0.4064) (layer F.Cu) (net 18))
 (via (at 78.232 50.546) (size 0.9) (drill 0.4) (layers F.Cu B.Cu) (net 18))
 (segment (start 78.232 50.419) (end 78.232 50.546) (width 0.4064) (layer F.Cu) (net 18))
 (segment (start 79.375 49.403) (end 79.375 46.99) (width 0.4064) (layer B.Cu) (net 18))
 (segment (start 78.232 50.546) (end 79.375 49.403) (width 0.4064) (layer B.Cu) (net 18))
 (via (at 79.375 46.99) (size 0.9) (drill 0.4) (layers F.Cu B.Cu) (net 18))
 (via (at 57.15 49.911) (size 0.9) (drill 0.4) (layers F.Cu B.Cu) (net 19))
 (segment (start 57.15 49.911) (end 57.15 51.177) (width 0.4064) (layer F.Cu) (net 19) (status 20))
 (segment (start 64.77 41.275) (end 63.373 42.672) (width 0.4064) (layer B.Cu) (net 19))
 (segment (start 73.152 41.275) (end 64.77 41.275) (width 0.4064) (layer B.Cu) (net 19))
 (segment (start 73.914 42.037) (end 73.152 41.275) (width 0.4064) (layer B.Cu) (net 19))
 (segment (start 73.914 43.688) (end 73.914 42.037) (width 0.4064) (layer B.Cu) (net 19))
 (segment (start 74.676 44.45) (end 73.914 43.688) (width 0.4064) (layer B.Cu) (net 19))
 (segment (start 63.373 42.672) (end 63.373 44.704) (width 0.4064) (layer B.Cu) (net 19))
 (segment (start 74.676 45.785) (end 74.676 44.45) (width 0.4064) (layer B.Cu) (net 19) (status 10))
 (segment (start 63.373 44.704) (end 60.579 47.498) (width 0.4064) (layer B.Cu) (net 19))
 (segment (start 60.579 47.498) (end 58.166 47.498) (width 0.4064) (layer B.Cu) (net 19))
 (segment (start 57.15 48.514) (end 57.15 49.911) (width 0.4064) (layer B.Cu) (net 19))
 (segment (start 58.166 47.498) (end 57.15 48.514) (width 0.4064) (layer B.Cu) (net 19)))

